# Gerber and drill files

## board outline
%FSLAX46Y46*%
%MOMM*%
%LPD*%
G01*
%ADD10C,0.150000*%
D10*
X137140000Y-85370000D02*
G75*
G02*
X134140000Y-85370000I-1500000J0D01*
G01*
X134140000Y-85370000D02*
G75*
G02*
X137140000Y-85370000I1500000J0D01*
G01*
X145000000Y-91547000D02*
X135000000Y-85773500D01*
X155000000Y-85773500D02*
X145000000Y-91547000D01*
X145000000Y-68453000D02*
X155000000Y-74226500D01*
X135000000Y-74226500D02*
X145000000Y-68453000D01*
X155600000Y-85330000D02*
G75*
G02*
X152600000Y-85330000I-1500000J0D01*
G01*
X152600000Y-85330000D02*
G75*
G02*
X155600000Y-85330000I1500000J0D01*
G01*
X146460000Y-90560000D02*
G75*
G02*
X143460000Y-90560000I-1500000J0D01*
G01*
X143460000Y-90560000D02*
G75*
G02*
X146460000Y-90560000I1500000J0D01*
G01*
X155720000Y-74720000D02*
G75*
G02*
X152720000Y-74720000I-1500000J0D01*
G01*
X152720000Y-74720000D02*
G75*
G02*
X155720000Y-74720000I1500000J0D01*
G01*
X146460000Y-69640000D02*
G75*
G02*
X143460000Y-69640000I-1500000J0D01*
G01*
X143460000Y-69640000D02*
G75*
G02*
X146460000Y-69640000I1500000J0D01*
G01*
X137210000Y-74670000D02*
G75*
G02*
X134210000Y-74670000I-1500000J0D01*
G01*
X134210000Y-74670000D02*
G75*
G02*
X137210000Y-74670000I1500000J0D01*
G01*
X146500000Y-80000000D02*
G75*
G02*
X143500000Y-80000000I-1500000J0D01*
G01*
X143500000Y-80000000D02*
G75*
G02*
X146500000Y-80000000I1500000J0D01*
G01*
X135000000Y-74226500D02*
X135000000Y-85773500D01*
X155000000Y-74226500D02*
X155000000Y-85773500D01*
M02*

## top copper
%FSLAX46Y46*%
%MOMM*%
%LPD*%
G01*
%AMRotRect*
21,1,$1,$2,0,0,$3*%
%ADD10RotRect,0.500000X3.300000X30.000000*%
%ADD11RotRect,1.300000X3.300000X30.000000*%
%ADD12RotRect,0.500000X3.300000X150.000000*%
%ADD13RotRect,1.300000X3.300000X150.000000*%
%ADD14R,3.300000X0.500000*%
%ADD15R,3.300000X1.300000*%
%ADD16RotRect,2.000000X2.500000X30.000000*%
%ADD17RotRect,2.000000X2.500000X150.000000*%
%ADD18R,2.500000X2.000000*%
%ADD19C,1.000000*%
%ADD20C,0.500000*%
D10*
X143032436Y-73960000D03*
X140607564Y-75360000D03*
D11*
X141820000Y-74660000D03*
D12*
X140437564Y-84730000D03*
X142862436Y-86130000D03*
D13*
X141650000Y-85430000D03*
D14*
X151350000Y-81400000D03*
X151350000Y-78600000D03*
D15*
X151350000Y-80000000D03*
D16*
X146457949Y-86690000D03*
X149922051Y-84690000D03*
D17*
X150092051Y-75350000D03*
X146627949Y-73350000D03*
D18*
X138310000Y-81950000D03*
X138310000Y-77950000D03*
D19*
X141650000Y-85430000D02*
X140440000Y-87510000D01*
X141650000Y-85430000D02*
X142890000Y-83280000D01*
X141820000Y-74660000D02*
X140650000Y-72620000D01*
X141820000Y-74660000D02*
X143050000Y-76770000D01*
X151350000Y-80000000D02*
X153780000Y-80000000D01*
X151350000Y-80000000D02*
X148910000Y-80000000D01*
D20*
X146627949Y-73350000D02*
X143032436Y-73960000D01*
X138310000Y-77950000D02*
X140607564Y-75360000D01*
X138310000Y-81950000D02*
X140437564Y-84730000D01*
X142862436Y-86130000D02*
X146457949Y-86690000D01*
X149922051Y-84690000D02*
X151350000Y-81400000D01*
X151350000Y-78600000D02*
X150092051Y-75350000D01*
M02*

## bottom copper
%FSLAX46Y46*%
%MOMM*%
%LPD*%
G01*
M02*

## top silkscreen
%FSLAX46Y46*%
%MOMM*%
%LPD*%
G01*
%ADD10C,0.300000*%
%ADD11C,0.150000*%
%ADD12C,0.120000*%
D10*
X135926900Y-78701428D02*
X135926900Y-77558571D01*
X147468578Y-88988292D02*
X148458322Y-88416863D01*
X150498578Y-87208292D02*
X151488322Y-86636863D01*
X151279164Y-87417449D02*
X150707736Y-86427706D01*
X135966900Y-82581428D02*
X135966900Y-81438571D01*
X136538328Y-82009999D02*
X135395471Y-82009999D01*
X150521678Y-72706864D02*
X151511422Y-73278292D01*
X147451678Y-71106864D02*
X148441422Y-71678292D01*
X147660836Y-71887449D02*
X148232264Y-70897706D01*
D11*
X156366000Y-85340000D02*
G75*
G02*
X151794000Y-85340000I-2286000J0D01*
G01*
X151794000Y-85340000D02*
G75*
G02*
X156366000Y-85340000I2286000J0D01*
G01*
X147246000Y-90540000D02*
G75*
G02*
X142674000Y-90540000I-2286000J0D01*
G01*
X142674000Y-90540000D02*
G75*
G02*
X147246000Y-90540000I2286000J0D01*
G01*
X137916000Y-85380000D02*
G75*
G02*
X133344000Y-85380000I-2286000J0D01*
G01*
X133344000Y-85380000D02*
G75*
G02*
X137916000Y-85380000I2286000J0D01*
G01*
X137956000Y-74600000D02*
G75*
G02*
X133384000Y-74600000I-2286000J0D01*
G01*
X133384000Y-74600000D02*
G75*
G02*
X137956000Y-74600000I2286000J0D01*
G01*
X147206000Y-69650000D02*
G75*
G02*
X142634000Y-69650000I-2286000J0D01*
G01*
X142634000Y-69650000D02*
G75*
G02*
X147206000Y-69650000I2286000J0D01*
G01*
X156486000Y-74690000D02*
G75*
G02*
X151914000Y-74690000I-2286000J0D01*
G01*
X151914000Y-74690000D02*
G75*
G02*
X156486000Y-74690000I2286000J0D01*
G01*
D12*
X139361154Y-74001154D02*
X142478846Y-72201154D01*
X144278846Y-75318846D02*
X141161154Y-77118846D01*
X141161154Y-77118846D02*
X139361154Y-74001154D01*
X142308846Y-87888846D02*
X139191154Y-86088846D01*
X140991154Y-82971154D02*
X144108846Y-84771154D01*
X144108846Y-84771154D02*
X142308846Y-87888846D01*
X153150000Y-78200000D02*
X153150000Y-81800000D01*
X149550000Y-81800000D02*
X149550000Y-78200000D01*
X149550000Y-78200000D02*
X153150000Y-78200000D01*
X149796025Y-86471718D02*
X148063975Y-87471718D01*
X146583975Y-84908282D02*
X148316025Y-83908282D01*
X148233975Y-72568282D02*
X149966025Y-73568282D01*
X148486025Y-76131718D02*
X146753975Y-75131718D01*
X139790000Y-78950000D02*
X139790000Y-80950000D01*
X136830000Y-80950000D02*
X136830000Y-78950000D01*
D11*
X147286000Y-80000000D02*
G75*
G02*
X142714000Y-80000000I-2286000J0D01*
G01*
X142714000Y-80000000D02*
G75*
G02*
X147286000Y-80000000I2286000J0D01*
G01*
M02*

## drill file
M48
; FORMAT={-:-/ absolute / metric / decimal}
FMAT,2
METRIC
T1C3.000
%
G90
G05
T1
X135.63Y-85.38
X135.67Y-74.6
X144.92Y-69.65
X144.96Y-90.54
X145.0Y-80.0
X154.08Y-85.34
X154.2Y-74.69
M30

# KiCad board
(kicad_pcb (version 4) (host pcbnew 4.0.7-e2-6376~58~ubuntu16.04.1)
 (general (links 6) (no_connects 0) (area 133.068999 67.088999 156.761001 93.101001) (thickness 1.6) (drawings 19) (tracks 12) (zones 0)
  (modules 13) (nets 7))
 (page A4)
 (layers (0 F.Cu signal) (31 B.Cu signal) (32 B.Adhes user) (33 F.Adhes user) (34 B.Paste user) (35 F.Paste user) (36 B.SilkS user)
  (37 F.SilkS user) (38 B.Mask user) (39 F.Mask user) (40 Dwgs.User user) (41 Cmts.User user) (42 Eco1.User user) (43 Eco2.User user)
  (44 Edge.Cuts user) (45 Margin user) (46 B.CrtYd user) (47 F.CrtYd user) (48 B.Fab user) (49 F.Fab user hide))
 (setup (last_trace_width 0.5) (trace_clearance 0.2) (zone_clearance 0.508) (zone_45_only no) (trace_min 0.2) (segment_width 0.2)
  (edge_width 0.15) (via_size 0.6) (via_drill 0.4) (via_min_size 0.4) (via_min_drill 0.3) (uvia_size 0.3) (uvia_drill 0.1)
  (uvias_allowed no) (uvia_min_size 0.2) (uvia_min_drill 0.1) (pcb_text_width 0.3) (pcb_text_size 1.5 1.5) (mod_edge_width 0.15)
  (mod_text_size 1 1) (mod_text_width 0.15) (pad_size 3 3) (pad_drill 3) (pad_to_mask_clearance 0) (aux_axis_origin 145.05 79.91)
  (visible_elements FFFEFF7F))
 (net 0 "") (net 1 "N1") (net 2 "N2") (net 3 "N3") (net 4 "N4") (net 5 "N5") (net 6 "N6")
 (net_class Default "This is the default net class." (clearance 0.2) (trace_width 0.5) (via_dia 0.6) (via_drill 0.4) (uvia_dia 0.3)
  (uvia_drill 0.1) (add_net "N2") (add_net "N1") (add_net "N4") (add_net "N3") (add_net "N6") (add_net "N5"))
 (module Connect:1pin (layer F.Cu) (at 154.08 85.34)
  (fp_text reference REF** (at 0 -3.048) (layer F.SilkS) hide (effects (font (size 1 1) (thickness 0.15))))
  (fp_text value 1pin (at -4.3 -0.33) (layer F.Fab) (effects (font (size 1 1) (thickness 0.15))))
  (fp_circle (center 0 0) (end 0 -2.286) (layer F.SilkS) (width 0.15))
  (pad "" np_thru_hole circle (at 0 0) (size 3 3) (drill 3) (layers *.Cu *.Mask)))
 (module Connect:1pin (layer F.Cu) (at 144.96 90.54)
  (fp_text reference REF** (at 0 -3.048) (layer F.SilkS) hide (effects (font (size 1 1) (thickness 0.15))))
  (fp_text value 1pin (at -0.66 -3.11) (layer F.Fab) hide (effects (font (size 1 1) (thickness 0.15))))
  (fp_circle (center 0 0) (end 0 -2.286) (layer F.SilkS) (width 0.15))
  (pad "" np_thru_hole circle (at 0 0) (size 3 3) (drill 3) (layers *.Cu *.Mask)))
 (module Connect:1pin (layer F.Cu) (at 135.63 85.38)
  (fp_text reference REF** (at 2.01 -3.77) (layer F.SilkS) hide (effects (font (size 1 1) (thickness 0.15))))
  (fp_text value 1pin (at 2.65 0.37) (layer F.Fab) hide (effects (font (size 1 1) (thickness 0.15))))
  (fp_circle (center 0 0) (end 0 -2.286) (layer F.SilkS) (width 0.15))
  (pad "" np_thru_hole circle (at 0 0) (size 3 3) (drill 3) (layers *.Cu *.Mask)))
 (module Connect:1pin (layer F.Cu) (at 135.67 74.6)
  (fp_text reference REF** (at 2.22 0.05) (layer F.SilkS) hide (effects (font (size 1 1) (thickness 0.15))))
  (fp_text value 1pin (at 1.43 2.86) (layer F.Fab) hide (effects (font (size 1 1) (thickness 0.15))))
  (fp_circle (center 0 0) (end 0 -2.286) (layer F.SilkS) (width 0.15))
  (pad "" np_thru_hole circle (at 0 0) (size 3 3) (drill 3) (layers *.Cu *.Mask)))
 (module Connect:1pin (layer F.Cu) (at 144.92 69.65)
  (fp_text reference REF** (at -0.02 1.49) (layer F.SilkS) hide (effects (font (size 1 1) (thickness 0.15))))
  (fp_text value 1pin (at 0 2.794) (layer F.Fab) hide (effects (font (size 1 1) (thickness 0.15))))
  (fp_circle (center 0 0) (end 0 -2.286) (layer F.SilkS) (width 0.15))
  (pad "" np_thru_hole circle (at 0 0) (size 3 3) (drill 3) (layers *.Cu *.Mask)))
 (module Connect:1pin (layer F.Cu) (at 154.2 74.69)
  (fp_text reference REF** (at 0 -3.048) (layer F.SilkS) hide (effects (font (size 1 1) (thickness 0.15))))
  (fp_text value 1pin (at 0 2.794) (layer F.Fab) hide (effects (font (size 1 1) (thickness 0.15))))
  (fp_circle (center 0 0) (end 0 -2.286) (layer F.SilkS) (width 0.15))
  (pad "" np_thru_hole circle (at 0 0) (size 3 3) (drill 3) (layers *.Cu *.Mask)))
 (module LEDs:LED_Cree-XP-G (layer F.Cu) (at 141.82 74.66 30)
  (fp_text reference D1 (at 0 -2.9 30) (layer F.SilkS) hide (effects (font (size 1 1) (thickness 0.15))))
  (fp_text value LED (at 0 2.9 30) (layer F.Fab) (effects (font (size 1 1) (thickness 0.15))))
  (fp_line (start -1.8 -1.8) (end 1.8 -1.8) (layer F.SilkS) (width 0.12))
  (fp_line (start 1.8 1.8) (end -1.8 1.8) (layer F.SilkS) (width 0.12))
  (fp_line (start -1.8 1.8) (end -1.8 -1.8) (layer F.SilkS) (width 0.12))
  (pad 2 smd rect (at 1.4 0 30) (size 0.5 3.3) (layers F.Cu F.Paste F.Mask) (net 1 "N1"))
  (pad 1 smd rect (at -1.4 0 30) (size 0.5 3.3) (layers F.Cu F.Paste F.Mask) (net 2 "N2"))
  (pad 3 smd rect (at 0 0 30) (size 1.3 3.3) (layers F.Cu F.Mask))
  (pad 3 smd rect (at 0 0 30) (size 1.01 0.75) (layers F.Paste))
  (pad 3 smd rect (at 0 1 30) (size 1.01 0.75) (layers F.Paste))
  (pad 3 smd rect (at 0 -1 30) (size 1.01 0.75) (layers F.Paste)))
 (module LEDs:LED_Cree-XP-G (layer F.Cu) (at 141.65 85.43 150)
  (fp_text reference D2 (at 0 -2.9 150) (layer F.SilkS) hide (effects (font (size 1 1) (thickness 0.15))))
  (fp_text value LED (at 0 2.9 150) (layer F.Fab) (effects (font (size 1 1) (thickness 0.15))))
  (fp_line (start -1.8 -1.8) (end 1.8 -1.8) (layer F.SilkS) (width 0.12))
  (fp_line (start 1.8 1.8) (end -1.8 1.8) (layer F.SilkS) (width 0.12))
  (fp_line (start -1.8 1.8) (end -1.8 -1.8) (layer F.SilkS) (width 0.12))
  (pad 2 smd rect (at 1.4 0 150) (size 0.5 3.3) (layers F.Cu F.Paste F.Mask) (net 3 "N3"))
  (pad 1 smd rect (at -1.4 0 150) (size 0.5 3.3) (layers F.Cu F.Paste F.Mask) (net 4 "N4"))
  (pad 3 smd rect (at 0 0 150) (size 1.3 3.3) (layers F.Cu F.Mask))
  (pad 3 smd rect (at 0 0 150) (size 1.01 0.75) (layers F.Paste))
  (pad 3 smd rect (at 0 1 150) (size 1.01 0.75) (layers F.Paste))
  (pad 3 smd rect (at 0 -1 150) (size 1.01 0.75) (layers F.Paste)))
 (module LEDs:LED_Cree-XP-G (layer F.Cu) (at 151.35 80 270)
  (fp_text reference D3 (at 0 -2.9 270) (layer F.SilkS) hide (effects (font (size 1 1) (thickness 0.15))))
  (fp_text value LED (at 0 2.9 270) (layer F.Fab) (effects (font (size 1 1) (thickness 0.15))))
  (fp_line (start -1.8 -1.8) (end 1.8 -1.8) (layer F.SilkS) (width 0.12))
  (fp_line (start 1.8 1.8) (end -1.8 1.8) (layer F.SilkS) (width 0.12))
  (fp_line (start -1.8 1.8) (end -1.8 -1.8) (layer F.SilkS) (width 0.12))
  (pad 2 smd rect (at 1.4 0 270) (size 0.5 3.3) (layers F.Cu F.Paste F.Mask) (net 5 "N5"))
  (pad 1 smd rect (at -1.4 0 270) (size 0.5 3.3) (layers F.Cu F.Paste F.Mask) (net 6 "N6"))
  (pad 3 smd rect (at 0 0 270) (size 1.3 3.3) (layers F.Cu F.Mask))
  (pad 3 smd rect (at 0 0 270) (size 1.01 0.75) (layers F.Paste))
  (pad 3 smd rect (at 0 1 270) (size 1.01 0.75) (layers F.Paste))
  (pad 3 smd rect (at 0 -1 270) (size 1.01 0.75) (layers F.Paste)))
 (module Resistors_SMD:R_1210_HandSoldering (layer F.Cu) (at 148.19 85.69 30)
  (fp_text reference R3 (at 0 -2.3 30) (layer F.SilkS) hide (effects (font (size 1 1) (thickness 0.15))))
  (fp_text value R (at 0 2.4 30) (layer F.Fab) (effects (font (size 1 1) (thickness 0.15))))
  (fp_line (start 1 1.48) (end -1 1.48) (layer F.SilkS) (width 0.12))
  (fp_line (start -1 -1.48) (end 1 -1.48) (layer F.SilkS) (width 0.12))
  (pad 1 smd rect (at -2 0 30) (size 2 2.5) (layers F.Cu F.Paste F.Mask) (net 4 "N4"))
  (pad 2 smd rect (at 2 0 30) (size 2 2.5) (layers F.Cu F.Paste F.Mask) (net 5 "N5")))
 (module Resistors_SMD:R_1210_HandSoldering (layer F.Cu) (at 148.36 74.35 150)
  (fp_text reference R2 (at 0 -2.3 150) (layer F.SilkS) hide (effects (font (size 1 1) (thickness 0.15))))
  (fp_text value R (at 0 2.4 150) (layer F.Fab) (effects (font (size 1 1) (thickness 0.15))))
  (fp_line (start 1 1.48) (end -1 1.48) (layer F.SilkS) (width 0.12))
  (fp_line (start -1 -1.48) (end 1 -1.48) (layer F.SilkS) (width 0.12))
  (pad 1 smd rect (at -2 0 150) (size 2 2.5) (layers F.Cu F.Paste F.Mask) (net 6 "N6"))
  (pad 2 smd rect (at 2 0 150) (size 2 2.5) (layers F.Cu F.Paste F.Mask) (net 1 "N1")))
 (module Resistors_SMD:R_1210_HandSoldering (layer F.Cu) (at 138.31 79.95 90)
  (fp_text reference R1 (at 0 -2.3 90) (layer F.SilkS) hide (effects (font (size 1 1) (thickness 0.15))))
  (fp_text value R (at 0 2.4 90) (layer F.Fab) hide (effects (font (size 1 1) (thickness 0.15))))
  (fp_line (start 1 1.48) (end -1 1.48) (layer F.SilkS) (width 0.12))
  (fp_line (start -1 -1.48) (end 1 -1.48) (layer F.SilkS) (width 0.12))
  (pad 1 smd rect (at -2 0 90) (size 2 2.5) (layers F.Cu F.Paste F.Mask) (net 3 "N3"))
  (pad 2 smd rect (at 2 0 90) (size 2 2.5) (layers F.Cu F.Paste F.Mask) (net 2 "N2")))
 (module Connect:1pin (layer F.Cu) (at 145 80)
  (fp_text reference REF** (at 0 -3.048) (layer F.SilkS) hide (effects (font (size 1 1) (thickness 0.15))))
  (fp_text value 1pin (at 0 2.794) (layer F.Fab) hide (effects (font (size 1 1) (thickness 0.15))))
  (fp_circle (center 0 0) (end 0 -2.286) (layer F.SilkS) (width 0.15))
  (pad "" np_thru_hole circle (at 0 0) (size 3 3) (drill 3) (layers *.Cu *.Mask)))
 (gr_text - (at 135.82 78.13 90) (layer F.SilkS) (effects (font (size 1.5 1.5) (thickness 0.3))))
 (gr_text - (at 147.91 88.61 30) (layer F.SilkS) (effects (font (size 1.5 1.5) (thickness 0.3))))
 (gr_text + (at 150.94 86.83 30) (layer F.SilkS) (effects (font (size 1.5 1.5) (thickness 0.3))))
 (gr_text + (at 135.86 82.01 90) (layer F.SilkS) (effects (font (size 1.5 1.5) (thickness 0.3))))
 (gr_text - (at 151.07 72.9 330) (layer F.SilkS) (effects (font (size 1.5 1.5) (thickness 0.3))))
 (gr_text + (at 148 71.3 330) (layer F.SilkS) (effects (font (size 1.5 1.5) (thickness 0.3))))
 (gr_circle (center 135.64 85.37) (end 134.14 85.37) (layer Edge.Cuts) (width 0.15))
 (gr_line (start 145 91.547) (end 135 85.7735) (angle 90) (layer Edge.Cuts) (width 0.15))
 (gr_line (start 155 85.7735) (end 145 91.547) (angle 90) (layer Edge.Cuts) (width 0.15))
 (gr_line (start 145 68.453) (end 155 74.2265) (angle 90) (layer Edge.Cuts) (width 0.15))
 (gr_line (start 135 74.2265) (end 145 68.453) (angle 90) (layer Edge.Cuts) (width 0.15))
 (gr_circle (center 154.1 85.33) (end 152.6 85.33) (layer Edge.Cuts) (width 0.15))
 (gr_circle (center 144.96 90.56) (end 143.46 90.56) (layer Edge.Cuts) (width 0.15))
 (gr_circle (center 154.22 74.72) (end 152.72 74.72) (layer Edge.Cuts) (width 0.15))
 (gr_circle (center 144.96 69.64) (end 143.46 69.64) (layer Edge.Cuts) (width 0.15))
 (gr_circle (center 135.71 74.67) (end 134.21 74.67) (layer Edge.Cuts) (width 0.15))
 (gr_circle (center 145 80) (end 143.5 80) (layer Edge.Cuts) (width 0.15))
 (gr_line (start 135 74.2265) (end 135 85.7735) (angle 90) (layer Edge.Cuts) (width 0.15))
 (gr_line (start 155 74.2265) (end 155 85.7735) (angle 90) (layer Edge.Cuts) (width 0.15))
 (segment (start 141.65 85.43) (end 140.44 87.51) (width 1) (layer F.Cu) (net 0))
 (segment (start 141.65 85.43) (end 142.89 83.28) (width 1) (layer F.Cu) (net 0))
 (segment (start 141.82 74.66) (end 140.65 72.62) (width 1) (layer F.Cu) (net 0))
 (segment (start 141.82 74.66) (end 143.05 76.77) (width 1) (layer F.Cu) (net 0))
 (segment (start 151.35 80) (end 153.78 80) (width 1) (layer F.Cu) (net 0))
 (segment (start 151.35 80) (end 148.91 80) (width 1) (layer F.Cu) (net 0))
 (segment (start 146.627949 73.35) (end 143.032436 73.96) (width 0.5) (layer F.Cu) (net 1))
 (segment (start 138.31 77.95) (end 140.607564 75.36) (width 0.5) (layer F.Cu) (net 2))
 (segment (start 138.31 81.95) (end 140.437564 84.73) (width 0.5) (layer F.Cu) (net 3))
 (segment (start 142.862436 86.13) (end 146.457949 86.69) (width 0.5) (layer F.Cu) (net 4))
 (segment (start 149.922051 84.69) (end 151.35 81.4) (width 0.5) (layer F.Cu) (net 5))
 (segment (start 151.35 78.6) (end 150.092051 75.35) (width 0.5) (layer F.Cu) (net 6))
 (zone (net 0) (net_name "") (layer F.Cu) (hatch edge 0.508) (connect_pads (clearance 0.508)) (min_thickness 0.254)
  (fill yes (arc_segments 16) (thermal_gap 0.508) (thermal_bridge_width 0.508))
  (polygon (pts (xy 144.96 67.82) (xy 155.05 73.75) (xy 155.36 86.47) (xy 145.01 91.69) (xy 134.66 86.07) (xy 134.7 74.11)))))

